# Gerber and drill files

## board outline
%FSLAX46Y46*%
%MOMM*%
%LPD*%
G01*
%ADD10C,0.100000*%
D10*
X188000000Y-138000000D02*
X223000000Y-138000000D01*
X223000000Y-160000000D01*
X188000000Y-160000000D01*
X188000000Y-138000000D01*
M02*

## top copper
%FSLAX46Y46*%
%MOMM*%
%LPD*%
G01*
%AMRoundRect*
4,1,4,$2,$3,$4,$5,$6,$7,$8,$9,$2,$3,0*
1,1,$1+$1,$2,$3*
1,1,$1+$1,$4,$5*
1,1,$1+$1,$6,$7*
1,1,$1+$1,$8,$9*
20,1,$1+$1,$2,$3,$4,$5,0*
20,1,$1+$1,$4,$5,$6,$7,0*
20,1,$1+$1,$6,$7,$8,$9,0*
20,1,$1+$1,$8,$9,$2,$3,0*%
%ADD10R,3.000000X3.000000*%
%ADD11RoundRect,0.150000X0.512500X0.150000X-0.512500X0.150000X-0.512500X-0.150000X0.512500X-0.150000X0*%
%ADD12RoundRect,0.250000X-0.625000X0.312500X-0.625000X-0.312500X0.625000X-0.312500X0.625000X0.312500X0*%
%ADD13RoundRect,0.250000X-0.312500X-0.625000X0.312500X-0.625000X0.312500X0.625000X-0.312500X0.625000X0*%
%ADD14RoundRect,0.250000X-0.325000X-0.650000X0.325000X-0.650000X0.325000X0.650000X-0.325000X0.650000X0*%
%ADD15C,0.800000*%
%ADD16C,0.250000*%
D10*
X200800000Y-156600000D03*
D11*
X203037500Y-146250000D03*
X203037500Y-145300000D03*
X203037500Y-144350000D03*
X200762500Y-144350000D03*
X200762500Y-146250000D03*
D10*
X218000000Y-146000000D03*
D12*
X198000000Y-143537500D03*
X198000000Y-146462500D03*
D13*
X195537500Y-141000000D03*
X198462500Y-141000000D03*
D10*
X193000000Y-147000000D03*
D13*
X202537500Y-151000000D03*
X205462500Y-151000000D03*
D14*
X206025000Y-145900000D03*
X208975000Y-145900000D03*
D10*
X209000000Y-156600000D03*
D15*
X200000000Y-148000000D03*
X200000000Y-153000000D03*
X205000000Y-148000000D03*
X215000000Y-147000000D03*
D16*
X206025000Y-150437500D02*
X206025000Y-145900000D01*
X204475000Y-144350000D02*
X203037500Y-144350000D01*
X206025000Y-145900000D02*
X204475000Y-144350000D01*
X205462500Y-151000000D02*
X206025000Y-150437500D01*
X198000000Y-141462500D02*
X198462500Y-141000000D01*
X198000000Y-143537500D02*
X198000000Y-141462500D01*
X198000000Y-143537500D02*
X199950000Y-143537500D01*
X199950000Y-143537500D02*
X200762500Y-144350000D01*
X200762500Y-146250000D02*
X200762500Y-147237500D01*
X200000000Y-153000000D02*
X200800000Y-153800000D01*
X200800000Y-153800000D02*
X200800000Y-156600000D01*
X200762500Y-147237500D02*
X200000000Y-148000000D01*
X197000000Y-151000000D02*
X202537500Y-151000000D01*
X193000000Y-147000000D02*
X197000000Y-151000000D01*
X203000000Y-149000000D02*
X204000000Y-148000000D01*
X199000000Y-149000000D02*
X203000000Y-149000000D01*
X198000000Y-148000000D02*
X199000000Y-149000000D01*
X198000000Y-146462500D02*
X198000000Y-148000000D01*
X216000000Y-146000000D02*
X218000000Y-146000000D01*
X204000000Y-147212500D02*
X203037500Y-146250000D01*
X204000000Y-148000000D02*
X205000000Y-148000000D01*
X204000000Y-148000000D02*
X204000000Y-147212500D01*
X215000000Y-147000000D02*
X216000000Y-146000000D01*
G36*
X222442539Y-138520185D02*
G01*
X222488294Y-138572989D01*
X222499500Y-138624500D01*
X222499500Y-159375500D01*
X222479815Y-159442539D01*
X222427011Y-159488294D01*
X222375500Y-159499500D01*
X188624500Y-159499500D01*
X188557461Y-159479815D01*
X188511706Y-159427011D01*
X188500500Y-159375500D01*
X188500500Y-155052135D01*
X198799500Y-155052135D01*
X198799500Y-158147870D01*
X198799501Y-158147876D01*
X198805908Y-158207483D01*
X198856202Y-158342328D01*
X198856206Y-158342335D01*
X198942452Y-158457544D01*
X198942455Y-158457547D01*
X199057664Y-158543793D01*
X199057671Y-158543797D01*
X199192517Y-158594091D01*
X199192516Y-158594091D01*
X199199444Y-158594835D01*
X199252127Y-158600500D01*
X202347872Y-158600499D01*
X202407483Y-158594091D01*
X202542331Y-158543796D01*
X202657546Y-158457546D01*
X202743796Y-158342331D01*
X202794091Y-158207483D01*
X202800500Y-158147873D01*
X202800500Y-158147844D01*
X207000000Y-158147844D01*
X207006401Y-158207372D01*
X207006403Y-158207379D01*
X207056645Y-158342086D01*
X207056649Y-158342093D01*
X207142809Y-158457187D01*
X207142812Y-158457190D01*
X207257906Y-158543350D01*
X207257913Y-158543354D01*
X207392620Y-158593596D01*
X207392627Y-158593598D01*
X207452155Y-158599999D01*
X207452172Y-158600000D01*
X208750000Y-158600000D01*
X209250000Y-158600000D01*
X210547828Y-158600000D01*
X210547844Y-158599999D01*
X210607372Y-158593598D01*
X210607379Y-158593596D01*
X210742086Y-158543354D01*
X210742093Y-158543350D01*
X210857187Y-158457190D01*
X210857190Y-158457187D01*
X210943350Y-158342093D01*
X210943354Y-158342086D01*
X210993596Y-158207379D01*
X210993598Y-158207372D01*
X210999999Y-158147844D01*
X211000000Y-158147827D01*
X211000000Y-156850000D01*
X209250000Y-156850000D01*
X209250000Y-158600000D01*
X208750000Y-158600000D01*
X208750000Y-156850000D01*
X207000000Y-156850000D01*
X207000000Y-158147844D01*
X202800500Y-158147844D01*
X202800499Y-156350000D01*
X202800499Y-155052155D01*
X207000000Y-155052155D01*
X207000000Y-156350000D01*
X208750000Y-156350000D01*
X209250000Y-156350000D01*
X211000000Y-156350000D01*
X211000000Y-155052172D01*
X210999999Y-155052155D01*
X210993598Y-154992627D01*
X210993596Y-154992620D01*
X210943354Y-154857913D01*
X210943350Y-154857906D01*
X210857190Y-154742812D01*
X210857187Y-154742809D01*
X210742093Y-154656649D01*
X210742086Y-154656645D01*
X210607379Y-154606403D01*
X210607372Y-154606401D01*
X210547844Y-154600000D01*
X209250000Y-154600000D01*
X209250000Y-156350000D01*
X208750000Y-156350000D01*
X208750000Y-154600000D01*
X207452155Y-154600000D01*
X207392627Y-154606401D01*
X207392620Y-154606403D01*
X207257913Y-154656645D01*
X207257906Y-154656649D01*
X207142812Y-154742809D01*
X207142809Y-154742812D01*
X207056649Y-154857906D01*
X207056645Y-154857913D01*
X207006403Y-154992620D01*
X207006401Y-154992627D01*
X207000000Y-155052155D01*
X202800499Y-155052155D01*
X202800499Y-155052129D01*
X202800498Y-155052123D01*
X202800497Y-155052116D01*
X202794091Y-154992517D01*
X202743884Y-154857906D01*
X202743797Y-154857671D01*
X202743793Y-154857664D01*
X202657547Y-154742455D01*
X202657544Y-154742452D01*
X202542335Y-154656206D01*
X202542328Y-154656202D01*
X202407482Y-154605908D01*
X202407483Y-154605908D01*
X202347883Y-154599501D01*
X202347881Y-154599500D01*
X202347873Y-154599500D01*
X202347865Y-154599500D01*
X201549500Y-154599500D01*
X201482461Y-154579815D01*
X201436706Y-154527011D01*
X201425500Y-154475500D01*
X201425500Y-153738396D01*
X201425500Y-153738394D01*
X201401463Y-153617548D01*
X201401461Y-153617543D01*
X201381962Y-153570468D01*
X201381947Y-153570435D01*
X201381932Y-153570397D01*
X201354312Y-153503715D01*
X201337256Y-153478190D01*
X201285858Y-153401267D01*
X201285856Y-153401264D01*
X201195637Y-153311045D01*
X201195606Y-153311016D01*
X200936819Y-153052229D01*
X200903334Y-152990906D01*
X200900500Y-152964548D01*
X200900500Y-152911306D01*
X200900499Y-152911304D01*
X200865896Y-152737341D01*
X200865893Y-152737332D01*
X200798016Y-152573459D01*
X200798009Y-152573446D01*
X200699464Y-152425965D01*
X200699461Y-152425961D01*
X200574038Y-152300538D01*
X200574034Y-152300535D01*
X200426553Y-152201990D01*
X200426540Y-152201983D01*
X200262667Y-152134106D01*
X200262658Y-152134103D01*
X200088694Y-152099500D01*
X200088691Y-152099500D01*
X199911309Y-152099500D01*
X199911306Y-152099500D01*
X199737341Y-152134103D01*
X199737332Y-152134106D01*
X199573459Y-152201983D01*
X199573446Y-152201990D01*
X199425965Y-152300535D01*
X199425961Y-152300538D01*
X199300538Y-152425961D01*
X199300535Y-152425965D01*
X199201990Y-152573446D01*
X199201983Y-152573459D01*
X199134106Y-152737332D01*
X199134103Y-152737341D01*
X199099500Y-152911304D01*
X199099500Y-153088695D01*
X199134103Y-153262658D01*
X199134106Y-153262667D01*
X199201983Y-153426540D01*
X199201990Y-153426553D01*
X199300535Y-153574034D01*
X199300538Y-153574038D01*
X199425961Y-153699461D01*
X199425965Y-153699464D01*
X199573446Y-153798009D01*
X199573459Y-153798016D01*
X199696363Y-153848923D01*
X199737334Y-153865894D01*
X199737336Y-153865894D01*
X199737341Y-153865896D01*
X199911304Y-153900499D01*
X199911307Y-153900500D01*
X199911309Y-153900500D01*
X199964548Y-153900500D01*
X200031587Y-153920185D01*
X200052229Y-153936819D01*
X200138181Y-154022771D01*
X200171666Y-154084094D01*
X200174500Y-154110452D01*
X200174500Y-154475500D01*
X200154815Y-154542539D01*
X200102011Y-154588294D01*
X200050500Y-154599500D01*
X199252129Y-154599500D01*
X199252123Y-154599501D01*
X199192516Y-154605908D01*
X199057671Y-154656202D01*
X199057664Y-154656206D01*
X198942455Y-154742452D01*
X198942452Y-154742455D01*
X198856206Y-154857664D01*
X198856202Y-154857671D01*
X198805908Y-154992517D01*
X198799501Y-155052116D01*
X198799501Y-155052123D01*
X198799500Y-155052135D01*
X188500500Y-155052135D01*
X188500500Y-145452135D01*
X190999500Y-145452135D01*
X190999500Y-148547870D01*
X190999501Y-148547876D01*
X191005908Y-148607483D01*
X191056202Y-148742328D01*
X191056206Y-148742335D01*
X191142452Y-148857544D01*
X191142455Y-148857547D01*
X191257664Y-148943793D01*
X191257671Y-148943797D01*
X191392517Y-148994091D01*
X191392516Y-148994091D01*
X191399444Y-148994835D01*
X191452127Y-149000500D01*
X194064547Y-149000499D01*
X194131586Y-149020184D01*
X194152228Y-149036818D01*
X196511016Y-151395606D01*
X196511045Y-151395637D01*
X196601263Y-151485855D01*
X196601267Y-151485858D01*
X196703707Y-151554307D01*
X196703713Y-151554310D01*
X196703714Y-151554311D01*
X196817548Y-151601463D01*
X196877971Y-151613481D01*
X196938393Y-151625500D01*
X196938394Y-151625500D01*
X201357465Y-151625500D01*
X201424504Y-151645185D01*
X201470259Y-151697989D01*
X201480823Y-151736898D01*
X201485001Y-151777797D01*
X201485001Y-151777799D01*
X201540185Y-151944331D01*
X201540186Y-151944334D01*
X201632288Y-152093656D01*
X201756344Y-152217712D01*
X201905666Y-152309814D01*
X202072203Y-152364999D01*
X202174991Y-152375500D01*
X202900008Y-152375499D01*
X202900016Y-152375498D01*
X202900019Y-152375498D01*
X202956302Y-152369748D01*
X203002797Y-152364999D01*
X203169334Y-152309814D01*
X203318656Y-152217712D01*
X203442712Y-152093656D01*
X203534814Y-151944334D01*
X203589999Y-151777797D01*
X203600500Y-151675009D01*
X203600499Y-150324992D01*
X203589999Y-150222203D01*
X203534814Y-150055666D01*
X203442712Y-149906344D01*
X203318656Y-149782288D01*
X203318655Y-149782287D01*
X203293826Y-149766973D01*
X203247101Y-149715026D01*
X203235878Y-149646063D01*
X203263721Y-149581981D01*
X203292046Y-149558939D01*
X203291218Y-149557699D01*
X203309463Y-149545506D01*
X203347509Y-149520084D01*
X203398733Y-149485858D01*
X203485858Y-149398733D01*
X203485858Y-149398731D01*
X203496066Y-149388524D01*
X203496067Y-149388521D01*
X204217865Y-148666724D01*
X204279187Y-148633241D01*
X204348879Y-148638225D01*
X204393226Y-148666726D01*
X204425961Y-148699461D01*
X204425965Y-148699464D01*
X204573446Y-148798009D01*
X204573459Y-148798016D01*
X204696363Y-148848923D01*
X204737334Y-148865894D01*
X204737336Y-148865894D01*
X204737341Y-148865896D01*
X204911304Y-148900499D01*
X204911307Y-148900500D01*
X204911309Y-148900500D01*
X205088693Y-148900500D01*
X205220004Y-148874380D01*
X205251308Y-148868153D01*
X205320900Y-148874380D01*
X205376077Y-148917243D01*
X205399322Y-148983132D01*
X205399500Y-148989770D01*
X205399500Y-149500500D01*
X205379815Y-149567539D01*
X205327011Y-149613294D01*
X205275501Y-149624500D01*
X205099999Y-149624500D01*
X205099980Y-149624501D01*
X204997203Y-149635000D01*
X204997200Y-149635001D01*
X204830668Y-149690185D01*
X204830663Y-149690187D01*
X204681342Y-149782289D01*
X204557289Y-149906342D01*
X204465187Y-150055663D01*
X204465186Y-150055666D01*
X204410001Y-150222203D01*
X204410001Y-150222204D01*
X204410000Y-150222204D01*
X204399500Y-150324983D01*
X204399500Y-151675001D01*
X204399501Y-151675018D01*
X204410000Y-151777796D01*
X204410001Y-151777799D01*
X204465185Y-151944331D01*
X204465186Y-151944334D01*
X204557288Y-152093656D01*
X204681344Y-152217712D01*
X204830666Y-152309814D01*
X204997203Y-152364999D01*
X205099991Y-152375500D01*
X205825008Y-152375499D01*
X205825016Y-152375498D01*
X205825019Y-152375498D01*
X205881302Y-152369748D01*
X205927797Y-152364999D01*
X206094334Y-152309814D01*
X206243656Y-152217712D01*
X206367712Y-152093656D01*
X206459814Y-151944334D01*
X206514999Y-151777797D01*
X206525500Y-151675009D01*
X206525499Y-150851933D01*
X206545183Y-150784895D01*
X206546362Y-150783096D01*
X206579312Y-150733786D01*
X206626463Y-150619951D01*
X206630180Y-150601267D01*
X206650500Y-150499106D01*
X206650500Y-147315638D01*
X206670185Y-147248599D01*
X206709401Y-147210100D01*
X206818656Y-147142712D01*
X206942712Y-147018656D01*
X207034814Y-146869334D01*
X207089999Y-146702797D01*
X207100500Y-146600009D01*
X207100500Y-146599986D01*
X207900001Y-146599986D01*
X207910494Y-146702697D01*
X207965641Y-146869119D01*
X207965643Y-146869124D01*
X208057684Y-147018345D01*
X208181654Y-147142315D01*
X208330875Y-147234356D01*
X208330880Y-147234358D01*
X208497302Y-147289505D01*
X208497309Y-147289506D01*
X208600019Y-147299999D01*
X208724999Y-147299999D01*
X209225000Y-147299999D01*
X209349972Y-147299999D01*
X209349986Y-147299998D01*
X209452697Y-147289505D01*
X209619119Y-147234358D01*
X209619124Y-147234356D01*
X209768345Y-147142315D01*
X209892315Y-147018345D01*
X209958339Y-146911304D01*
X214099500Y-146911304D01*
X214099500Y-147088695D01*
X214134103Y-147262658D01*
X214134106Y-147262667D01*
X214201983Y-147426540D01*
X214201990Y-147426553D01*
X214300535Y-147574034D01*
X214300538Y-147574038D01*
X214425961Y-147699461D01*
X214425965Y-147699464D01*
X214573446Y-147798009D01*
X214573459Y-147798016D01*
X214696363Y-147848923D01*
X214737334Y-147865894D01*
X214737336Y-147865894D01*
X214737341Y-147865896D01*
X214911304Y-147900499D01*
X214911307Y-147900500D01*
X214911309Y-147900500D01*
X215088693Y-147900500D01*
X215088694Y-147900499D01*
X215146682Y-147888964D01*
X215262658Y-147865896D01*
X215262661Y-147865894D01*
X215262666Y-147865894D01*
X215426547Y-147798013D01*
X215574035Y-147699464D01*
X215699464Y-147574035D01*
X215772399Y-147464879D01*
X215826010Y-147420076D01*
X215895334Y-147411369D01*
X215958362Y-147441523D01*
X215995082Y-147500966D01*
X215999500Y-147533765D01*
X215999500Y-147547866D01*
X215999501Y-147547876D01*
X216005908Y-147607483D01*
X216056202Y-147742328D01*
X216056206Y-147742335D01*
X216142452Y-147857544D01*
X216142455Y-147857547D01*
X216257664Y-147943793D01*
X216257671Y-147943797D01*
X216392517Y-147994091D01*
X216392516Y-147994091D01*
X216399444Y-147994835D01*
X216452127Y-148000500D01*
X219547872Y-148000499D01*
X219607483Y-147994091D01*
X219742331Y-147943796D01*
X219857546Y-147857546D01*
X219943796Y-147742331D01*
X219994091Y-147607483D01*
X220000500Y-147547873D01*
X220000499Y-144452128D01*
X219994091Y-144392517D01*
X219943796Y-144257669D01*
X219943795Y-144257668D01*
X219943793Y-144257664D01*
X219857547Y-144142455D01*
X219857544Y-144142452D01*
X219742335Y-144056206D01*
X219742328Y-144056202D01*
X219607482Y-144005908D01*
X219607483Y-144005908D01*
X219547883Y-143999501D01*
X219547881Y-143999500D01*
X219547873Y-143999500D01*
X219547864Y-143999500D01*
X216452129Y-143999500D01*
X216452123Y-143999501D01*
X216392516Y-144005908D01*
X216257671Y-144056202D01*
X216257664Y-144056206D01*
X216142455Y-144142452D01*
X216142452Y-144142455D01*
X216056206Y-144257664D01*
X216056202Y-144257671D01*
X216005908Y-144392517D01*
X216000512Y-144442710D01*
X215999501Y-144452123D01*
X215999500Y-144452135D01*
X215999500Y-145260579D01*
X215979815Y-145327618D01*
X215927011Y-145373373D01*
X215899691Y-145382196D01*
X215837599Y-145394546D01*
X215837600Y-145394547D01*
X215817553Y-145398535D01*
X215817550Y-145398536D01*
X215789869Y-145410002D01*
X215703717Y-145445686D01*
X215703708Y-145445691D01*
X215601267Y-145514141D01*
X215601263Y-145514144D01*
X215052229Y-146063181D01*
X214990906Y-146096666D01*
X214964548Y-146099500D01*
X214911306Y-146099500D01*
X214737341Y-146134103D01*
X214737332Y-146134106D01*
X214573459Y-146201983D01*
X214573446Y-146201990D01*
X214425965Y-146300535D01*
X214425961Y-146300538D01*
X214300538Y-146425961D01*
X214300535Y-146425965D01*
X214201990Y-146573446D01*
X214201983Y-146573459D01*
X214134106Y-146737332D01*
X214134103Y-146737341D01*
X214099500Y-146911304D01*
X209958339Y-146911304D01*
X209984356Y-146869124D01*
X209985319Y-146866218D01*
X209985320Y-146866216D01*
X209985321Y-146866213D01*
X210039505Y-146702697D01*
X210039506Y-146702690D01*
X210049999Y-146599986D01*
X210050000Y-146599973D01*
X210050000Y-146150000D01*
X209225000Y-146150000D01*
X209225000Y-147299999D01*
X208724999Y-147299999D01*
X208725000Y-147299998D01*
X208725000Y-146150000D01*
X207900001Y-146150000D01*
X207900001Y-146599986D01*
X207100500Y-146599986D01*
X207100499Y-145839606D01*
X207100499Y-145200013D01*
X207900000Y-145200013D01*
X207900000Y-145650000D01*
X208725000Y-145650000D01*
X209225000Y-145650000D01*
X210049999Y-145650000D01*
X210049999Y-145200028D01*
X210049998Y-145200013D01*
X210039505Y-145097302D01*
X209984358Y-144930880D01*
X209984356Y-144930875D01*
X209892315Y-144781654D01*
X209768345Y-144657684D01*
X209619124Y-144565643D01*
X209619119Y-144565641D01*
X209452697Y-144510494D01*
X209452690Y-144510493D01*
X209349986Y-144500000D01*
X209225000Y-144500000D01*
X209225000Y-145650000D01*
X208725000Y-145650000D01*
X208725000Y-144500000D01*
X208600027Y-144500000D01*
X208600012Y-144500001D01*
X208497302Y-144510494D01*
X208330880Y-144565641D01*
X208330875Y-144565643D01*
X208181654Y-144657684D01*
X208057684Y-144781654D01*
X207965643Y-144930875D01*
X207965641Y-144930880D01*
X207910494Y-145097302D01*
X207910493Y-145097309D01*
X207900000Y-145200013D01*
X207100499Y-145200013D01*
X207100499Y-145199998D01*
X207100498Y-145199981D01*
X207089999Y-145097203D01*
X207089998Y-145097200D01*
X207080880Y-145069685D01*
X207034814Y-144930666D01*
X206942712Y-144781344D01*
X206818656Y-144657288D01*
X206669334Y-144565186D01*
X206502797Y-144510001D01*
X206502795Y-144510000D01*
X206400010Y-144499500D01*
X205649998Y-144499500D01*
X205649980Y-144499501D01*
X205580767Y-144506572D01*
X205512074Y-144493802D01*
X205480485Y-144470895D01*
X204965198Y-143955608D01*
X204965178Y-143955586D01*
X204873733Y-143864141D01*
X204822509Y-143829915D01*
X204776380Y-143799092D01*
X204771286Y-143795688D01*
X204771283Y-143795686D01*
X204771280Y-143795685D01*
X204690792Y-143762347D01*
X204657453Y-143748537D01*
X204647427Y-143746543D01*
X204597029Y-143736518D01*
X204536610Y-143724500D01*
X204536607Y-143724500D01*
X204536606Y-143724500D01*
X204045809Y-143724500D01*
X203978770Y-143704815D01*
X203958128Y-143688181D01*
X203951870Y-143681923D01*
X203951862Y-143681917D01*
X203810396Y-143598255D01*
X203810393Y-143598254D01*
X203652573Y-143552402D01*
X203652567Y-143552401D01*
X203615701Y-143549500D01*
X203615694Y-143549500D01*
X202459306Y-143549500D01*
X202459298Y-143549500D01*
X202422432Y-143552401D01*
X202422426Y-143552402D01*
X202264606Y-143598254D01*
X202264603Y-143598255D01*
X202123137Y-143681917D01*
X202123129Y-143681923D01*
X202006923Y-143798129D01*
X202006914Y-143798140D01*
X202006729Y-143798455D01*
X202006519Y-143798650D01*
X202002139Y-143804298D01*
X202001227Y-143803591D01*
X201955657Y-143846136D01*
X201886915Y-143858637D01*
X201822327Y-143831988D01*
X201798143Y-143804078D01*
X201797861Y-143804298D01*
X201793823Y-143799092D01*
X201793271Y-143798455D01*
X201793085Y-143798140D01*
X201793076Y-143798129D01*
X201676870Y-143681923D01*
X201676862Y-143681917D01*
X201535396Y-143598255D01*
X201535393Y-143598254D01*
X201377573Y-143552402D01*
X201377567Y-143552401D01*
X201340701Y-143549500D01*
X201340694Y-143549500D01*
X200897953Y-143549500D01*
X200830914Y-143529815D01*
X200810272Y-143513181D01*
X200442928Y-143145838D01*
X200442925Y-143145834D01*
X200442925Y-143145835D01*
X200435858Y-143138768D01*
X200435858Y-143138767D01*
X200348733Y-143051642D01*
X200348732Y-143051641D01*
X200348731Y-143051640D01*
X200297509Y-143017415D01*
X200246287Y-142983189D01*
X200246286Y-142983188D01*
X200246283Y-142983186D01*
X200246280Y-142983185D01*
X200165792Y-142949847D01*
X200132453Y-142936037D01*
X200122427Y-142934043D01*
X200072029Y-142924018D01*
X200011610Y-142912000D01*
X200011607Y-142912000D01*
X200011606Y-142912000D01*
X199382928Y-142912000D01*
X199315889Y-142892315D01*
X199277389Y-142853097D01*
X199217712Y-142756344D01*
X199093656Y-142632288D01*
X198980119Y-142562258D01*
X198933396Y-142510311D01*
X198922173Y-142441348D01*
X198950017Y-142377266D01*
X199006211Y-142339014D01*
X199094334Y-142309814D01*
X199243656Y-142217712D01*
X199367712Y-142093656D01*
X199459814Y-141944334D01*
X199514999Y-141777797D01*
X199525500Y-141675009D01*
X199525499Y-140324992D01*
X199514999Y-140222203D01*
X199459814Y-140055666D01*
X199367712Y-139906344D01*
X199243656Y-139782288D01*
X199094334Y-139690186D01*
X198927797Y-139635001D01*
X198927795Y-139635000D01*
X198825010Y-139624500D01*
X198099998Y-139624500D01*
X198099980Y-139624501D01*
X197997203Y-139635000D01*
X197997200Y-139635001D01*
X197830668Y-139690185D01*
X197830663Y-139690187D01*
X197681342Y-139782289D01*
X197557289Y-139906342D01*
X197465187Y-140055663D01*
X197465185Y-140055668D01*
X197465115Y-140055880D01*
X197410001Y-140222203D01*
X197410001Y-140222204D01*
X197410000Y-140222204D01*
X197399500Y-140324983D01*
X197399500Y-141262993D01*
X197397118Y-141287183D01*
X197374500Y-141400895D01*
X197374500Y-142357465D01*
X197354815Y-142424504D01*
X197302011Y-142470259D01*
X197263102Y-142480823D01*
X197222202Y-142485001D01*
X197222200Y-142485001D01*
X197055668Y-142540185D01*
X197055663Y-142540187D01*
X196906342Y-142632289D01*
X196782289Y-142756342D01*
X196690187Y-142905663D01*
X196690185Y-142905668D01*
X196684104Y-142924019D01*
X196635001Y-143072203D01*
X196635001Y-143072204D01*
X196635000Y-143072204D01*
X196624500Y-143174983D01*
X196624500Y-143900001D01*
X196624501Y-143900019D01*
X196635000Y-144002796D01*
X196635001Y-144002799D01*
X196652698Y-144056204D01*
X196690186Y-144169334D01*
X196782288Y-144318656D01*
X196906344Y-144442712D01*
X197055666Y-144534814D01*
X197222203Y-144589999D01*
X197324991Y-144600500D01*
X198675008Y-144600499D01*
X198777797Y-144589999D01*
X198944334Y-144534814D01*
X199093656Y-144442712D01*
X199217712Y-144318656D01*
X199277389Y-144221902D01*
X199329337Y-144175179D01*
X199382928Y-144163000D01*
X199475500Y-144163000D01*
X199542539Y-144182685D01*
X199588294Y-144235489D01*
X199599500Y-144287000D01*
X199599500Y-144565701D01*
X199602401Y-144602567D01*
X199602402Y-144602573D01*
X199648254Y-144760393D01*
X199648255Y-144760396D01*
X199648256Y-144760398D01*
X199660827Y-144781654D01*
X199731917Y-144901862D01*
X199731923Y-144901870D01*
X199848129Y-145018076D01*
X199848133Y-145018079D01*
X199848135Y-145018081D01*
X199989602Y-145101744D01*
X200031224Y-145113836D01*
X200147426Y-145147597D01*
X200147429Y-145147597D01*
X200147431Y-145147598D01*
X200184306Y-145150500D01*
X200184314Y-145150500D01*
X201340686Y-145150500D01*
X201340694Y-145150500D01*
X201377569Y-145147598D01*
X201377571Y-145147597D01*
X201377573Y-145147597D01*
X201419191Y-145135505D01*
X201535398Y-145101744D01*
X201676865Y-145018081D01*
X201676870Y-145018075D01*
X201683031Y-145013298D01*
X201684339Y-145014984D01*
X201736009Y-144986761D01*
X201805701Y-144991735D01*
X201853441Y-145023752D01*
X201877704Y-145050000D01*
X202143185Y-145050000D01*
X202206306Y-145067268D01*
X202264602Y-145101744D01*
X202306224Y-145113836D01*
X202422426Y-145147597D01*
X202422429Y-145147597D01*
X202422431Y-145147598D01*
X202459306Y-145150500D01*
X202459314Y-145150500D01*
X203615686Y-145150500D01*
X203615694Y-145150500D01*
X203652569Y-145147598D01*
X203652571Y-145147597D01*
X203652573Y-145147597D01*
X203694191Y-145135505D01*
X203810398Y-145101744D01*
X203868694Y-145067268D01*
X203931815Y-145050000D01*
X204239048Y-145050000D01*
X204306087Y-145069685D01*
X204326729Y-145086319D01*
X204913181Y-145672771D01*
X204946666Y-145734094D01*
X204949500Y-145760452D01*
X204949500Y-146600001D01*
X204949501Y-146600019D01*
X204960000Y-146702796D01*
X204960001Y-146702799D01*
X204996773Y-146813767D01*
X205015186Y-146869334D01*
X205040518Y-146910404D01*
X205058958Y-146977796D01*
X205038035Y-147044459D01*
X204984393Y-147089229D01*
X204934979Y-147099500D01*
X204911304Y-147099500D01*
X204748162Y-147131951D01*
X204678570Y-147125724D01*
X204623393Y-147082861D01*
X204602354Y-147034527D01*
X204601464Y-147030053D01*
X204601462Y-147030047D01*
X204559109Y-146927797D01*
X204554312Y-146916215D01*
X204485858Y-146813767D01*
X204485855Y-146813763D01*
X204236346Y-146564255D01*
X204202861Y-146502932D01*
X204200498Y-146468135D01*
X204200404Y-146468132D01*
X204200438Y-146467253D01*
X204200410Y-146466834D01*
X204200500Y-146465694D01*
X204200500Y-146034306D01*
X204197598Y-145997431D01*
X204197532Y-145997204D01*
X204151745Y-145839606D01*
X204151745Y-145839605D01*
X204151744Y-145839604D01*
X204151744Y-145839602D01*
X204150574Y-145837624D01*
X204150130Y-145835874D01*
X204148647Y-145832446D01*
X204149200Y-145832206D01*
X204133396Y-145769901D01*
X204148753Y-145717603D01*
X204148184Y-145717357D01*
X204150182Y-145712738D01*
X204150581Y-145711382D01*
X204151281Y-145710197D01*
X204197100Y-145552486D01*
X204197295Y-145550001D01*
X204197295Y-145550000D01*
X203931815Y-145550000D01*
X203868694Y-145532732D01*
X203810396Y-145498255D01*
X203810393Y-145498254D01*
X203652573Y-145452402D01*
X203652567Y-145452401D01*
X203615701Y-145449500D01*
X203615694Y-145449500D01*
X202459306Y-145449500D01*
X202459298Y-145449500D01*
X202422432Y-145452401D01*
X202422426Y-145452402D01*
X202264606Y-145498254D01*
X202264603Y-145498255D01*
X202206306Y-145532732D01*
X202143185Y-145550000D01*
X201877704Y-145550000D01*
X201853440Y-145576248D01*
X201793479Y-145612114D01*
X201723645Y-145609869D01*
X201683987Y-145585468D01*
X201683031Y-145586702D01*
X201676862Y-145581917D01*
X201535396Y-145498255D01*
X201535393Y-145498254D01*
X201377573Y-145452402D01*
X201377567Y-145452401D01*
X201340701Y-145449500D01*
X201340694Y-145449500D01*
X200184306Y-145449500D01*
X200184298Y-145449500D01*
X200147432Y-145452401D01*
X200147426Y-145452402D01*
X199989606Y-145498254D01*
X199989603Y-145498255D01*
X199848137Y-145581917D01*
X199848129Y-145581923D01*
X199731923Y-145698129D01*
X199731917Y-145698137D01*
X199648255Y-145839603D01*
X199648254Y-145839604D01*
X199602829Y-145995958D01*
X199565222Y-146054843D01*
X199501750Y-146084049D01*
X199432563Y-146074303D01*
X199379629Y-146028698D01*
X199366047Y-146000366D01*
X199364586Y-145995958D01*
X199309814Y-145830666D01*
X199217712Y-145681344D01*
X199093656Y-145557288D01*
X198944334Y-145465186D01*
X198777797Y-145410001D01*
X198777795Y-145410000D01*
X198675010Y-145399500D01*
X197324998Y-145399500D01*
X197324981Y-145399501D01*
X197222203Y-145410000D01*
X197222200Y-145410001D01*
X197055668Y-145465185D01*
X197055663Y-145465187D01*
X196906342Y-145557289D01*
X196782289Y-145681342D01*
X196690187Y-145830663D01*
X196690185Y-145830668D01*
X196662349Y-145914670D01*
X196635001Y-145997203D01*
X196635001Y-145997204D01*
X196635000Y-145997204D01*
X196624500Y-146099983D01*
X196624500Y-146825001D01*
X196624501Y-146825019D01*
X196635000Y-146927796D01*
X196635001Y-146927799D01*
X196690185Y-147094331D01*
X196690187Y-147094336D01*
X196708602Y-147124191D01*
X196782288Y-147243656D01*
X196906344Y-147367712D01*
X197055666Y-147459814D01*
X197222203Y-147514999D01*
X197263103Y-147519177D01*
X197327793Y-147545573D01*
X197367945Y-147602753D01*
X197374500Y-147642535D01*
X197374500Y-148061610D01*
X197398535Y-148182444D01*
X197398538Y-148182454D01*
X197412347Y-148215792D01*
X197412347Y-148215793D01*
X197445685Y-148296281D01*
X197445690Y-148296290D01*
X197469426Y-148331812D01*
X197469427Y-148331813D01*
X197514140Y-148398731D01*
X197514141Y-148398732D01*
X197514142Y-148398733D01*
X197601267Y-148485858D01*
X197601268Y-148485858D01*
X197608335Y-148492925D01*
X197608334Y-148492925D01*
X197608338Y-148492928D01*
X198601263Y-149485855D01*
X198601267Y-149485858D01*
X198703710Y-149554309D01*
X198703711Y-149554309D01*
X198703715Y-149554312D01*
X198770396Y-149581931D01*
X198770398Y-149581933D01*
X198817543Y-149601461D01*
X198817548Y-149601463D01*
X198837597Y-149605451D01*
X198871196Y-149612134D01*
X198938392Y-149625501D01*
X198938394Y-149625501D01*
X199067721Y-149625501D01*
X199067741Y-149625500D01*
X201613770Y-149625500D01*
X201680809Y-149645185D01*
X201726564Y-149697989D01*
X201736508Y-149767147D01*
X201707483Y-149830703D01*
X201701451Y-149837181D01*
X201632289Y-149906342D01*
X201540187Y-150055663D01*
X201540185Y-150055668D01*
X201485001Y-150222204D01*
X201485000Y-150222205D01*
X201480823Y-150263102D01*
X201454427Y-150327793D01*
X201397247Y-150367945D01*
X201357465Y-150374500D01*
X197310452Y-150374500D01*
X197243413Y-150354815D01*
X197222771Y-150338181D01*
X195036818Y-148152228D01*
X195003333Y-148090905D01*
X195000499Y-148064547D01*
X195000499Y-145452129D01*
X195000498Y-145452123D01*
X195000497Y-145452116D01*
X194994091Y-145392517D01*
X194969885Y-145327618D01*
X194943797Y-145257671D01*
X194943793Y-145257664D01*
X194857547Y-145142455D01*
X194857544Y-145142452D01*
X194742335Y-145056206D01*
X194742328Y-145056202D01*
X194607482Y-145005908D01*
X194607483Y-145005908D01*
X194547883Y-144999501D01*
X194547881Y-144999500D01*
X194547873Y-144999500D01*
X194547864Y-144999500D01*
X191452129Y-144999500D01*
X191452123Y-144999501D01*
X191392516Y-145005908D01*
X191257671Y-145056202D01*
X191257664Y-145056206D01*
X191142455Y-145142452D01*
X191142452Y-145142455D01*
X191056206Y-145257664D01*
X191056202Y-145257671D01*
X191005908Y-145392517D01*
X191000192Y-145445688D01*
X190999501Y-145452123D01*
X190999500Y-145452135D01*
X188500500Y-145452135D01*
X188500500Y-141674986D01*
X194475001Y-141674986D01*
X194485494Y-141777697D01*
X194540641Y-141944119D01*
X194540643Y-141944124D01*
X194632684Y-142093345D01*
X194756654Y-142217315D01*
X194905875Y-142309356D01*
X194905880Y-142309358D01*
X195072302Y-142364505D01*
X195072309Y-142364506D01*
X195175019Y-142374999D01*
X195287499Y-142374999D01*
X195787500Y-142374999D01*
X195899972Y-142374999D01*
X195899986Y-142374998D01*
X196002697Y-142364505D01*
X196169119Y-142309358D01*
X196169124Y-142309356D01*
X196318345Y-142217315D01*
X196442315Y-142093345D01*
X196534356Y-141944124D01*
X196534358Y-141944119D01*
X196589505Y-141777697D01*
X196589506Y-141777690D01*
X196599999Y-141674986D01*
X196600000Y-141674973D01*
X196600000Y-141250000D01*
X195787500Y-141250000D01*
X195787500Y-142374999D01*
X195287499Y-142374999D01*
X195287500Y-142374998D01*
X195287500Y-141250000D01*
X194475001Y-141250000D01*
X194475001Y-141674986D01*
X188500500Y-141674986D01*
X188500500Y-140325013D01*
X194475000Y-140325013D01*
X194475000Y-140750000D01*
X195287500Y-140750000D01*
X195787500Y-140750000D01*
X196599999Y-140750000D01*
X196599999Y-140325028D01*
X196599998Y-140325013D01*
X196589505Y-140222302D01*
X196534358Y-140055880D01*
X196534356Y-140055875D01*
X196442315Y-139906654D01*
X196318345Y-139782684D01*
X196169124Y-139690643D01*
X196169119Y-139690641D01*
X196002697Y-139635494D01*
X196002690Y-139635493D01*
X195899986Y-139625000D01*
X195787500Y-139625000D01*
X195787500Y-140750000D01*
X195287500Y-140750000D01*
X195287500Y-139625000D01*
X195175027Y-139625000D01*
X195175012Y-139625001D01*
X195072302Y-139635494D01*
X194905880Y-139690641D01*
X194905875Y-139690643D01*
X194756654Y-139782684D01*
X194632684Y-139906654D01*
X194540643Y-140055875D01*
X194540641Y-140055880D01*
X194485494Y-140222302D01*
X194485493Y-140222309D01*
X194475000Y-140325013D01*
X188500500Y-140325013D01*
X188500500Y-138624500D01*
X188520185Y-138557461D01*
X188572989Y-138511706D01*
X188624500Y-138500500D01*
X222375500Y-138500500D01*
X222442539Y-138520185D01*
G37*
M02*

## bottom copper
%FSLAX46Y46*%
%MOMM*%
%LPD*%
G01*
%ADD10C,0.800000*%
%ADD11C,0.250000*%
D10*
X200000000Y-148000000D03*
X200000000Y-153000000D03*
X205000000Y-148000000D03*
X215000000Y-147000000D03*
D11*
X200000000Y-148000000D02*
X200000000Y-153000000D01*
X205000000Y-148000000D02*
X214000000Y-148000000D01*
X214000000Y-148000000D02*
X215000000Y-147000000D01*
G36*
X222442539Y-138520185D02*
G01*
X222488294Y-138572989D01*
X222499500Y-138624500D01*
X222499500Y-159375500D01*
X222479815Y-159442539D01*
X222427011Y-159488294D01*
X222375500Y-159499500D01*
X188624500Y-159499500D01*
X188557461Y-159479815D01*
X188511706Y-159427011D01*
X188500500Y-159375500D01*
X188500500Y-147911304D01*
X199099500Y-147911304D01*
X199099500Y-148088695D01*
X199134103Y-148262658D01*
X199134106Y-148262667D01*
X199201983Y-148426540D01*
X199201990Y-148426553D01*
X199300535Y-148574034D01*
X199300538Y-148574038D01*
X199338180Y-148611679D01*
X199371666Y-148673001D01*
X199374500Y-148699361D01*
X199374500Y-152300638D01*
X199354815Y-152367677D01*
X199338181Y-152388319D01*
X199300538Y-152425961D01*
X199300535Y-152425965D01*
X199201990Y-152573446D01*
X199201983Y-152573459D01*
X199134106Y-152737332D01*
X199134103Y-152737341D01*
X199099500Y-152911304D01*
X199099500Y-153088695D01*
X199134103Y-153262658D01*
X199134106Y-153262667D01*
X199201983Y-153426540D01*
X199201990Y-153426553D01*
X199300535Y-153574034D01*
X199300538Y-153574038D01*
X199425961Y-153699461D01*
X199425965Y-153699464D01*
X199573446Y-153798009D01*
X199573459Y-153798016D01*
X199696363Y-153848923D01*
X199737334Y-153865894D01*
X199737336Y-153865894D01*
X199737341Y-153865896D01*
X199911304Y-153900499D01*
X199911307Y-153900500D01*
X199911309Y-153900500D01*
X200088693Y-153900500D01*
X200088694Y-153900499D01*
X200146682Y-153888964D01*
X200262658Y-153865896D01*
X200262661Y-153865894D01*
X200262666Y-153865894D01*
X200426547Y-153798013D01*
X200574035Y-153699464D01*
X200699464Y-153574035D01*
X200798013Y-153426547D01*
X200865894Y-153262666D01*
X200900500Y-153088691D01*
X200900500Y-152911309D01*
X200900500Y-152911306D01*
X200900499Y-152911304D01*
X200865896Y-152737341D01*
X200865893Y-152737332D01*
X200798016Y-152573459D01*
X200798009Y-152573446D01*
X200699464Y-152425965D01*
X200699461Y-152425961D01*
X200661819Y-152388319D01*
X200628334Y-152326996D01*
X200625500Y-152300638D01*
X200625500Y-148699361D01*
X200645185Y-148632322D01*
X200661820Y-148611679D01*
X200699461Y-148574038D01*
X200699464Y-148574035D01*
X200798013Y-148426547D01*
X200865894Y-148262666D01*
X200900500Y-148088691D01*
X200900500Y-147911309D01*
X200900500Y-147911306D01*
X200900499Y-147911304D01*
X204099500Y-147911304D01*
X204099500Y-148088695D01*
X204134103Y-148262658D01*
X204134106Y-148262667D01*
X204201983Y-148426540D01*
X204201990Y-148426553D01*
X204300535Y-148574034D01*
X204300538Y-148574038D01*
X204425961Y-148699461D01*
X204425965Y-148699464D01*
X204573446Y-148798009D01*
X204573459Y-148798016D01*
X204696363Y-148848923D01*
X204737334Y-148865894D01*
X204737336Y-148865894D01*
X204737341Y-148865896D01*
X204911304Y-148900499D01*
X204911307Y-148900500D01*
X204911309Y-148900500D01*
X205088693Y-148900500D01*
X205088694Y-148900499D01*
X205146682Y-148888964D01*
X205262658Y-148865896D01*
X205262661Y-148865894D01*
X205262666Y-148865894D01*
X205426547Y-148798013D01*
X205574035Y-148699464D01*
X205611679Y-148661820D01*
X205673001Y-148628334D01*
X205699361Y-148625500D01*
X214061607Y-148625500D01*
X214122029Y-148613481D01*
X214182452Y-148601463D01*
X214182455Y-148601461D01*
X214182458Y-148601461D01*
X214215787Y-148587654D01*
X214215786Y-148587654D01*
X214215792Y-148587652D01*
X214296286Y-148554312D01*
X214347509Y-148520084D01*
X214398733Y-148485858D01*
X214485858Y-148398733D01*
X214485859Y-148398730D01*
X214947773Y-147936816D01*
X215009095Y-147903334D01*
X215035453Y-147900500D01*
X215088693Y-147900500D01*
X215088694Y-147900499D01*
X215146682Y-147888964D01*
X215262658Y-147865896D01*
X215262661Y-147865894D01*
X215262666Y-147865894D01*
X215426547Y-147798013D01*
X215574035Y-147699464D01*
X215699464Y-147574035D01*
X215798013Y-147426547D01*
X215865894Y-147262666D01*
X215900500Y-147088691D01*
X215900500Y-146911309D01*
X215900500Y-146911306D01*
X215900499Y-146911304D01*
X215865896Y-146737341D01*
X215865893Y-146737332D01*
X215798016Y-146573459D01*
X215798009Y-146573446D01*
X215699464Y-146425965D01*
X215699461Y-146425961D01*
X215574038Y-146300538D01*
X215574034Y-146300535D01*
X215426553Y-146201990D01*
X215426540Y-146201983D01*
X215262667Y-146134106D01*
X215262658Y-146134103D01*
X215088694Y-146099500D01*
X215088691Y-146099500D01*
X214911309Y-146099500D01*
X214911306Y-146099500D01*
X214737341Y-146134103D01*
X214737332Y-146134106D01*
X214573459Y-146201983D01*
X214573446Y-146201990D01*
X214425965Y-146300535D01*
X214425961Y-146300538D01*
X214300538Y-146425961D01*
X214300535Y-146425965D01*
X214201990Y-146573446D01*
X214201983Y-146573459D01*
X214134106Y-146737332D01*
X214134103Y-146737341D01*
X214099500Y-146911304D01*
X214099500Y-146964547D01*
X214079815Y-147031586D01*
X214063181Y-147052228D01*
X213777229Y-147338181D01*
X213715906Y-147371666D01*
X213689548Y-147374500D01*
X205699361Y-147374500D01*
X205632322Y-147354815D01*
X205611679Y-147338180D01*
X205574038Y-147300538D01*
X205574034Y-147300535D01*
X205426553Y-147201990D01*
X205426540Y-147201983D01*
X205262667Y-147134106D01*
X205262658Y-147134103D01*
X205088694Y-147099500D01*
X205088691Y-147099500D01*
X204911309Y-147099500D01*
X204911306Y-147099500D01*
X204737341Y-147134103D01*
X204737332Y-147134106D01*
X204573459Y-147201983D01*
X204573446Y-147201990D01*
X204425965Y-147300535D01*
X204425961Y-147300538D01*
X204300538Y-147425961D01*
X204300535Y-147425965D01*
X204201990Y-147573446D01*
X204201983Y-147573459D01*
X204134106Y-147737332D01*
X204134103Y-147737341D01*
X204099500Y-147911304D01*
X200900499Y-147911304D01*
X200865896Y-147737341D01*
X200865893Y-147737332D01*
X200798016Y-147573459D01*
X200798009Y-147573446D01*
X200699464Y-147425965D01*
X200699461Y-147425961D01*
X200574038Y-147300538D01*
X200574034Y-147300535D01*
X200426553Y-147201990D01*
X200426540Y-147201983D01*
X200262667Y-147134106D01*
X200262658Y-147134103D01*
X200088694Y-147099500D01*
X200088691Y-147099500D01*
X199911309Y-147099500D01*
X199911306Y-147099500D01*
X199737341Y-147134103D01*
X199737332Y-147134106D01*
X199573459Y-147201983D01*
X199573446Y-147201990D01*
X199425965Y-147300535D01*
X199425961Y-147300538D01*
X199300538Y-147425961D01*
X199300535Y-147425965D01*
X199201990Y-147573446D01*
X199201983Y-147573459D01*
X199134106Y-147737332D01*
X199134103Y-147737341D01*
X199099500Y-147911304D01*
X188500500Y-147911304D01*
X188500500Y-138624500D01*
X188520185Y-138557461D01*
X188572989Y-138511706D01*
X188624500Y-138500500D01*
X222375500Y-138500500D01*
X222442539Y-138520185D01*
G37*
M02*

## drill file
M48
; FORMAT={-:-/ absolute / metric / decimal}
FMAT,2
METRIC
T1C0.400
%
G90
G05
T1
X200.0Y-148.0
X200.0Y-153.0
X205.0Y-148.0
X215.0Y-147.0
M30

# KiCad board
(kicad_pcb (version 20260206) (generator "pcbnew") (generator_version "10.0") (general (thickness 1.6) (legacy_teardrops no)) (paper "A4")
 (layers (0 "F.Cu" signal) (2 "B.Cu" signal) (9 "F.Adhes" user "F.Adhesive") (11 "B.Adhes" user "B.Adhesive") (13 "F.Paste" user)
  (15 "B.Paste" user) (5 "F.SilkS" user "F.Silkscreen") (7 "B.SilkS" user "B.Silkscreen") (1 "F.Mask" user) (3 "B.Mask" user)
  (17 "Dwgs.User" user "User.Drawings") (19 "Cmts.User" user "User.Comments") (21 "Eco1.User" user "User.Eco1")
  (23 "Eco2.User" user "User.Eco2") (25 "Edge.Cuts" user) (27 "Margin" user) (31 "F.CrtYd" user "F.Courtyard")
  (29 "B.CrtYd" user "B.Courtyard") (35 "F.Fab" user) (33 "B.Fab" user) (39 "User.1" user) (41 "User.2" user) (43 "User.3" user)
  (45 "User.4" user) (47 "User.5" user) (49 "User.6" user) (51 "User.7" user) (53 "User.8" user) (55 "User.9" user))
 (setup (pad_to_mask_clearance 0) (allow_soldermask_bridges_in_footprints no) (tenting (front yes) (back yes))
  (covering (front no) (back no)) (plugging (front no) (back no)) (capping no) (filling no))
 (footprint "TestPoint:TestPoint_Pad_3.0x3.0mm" (layer "F.Cu") (at 200.8 156.6)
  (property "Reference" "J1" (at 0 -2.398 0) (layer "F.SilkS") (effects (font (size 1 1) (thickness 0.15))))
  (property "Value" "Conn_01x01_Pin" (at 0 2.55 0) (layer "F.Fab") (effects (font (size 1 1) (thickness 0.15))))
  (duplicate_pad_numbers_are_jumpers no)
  (pad "1" smd rect (at 0 0) (size 3 3) (layers "F.Cu" "F.Mask") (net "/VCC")))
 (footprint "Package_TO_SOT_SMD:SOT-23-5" (layer "F.Cu") (at 201.9 145.3 180)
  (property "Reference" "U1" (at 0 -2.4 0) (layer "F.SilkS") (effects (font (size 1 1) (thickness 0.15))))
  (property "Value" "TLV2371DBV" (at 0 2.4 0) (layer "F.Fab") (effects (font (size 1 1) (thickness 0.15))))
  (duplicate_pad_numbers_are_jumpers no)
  (pad "1" smd roundrect (at -1.1375 -0.95 180) (size 1.325 0.6) (layers "F.Cu" "F.Mask" "F.Paste") (roundrect_rratio 0.25) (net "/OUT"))
  (pad "2" smd roundrect (at -1.1375 0 180) (size 1.325 0.6) (layers "F.Cu" "F.Mask" "F.Paste") (roundrect_rratio 0.25) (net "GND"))
  (pad "3" smd roundrect (at -1.1375 0.95 180) (size 1.325 0.6) (layers "F.Cu" "F.Mask" "F.Paste") (roundrect_rratio 0.25)
   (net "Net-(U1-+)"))
  (pad "4" smd roundrect (at 1.1375 0.95 180) (size 1.325 0.6) (layers "F.Cu" "F.Mask" "F.Paste") (roundrect_rratio 0.25) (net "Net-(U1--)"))
  (pad "5" smd roundrect (at 1.1375 -0.95 180) (size 1.325 0.6) (layers "F.Cu" "F.Mask" "F.Paste") (roundrect_rratio 0.25) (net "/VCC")))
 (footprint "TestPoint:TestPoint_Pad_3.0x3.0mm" (layer "F.Cu") (at 218 146)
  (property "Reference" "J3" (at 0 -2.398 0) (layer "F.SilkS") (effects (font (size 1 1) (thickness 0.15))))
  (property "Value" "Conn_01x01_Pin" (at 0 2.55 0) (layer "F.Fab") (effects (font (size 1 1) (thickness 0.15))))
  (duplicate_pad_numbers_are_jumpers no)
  (pad "1" smd rect (at 0 0) (size 3 3) (layers "F.Cu" "F.Mask") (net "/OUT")))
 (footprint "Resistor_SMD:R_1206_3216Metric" (layer "F.Cu") (at 198 145 -90)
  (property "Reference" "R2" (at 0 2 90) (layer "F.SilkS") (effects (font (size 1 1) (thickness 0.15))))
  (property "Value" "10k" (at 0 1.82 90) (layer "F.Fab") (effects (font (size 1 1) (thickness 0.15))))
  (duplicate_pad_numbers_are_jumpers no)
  (pad "1" smd roundrect (at -1.4625 0 270) (size 1.125 1.75) (layers "F.Cu" "F.Mask" "F.Paste") (roundrect_rratio 0.222222)
   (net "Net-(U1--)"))
  (pad "2" smd roundrect (at 1.4625 0 270) (size 1.125 1.75) (layers "F.Cu" "F.Mask" "F.Paste") (roundrect_rratio 0.222222) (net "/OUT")))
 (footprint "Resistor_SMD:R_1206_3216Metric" (layer "F.Cu") (at 197 141)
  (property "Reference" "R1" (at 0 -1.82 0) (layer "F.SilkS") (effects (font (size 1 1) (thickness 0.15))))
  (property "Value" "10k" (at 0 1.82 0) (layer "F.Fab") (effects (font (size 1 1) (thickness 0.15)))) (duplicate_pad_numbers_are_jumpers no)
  (pad "1" smd roundrect (at -1.4625 0) (size 1.125 1.75) (layers "F.Cu" "F.Mask" "F.Paste") (roundrect_rratio 0.222222) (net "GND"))
  (pad "2" smd roundrect (at 1.4625 0) (size 1.125 1.75) (layers "F.Cu" "F.Mask" "F.Paste") (roundrect_rratio 0.222222) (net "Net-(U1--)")))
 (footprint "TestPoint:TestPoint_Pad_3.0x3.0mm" (layer "F.Cu") (at 193 147)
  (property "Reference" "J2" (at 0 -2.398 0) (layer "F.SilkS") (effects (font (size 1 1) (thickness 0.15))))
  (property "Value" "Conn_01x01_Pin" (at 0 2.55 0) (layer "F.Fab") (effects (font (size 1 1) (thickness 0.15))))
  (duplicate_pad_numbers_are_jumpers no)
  (pad "1" smd rect (at 0 0) (size 3 3) (layers "F.Cu" "F.Mask") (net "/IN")))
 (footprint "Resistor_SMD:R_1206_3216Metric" (layer "F.Cu") (at 204 151)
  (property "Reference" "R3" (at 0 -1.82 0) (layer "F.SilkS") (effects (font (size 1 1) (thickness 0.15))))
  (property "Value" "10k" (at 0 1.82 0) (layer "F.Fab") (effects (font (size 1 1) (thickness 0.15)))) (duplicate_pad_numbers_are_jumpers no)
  (pad "1" smd roundrect (at -1.4625 0) (size 1.125 1.75) (layers "F.Cu" "F.Mask" "F.Paste") (roundrect_rratio 0.222222) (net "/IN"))
  (pad "2" smd roundrect (at 1.4625 0) (size 1.125 1.75) (layers "F.Cu" "F.Mask" "F.Paste") (roundrect_rratio 0.222222) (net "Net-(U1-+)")))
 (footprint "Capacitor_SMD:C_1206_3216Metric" (layer "F.Cu") (at 207.5 145.9)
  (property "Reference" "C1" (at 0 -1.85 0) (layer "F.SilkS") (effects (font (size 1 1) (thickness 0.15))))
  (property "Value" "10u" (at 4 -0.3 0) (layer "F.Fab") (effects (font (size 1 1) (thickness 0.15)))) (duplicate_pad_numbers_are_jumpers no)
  (pad "1" smd roundrect (at -1.475 0) (size 1.15 1.8) (layers "F.Cu" "F.Mask" "F.Paste") (roundrect_rratio 0.217391) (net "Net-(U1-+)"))
  (pad "2" smd roundrect (at 1.475 0) (size 1.15 1.8) (layers "F.Cu" "F.Mask" "F.Paste") (roundrect_rratio 0.217391) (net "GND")))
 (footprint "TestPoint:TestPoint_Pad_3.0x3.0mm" (layer "F.Cu") (at 209 156.6)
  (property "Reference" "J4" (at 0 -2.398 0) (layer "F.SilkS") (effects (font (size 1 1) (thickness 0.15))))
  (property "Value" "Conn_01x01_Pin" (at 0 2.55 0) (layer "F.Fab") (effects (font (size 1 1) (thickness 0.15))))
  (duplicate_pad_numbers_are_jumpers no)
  (pad "1" smd rect (at 0 0) (size 3 3) (layers "F.Cu" "F.Mask") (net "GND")))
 (gr_rect (start 188 138) (end 223 160) (stroke (width 0.1) (type default)) (fill no) (layer "Edge.Cuts"))
 (segment (start 206.025 150.4375) (end 206.025 145.9) (width 0.25) (layer "F.Cu") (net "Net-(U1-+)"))
 (segment (start 204.475 144.35) (end 203.0375 144.35) (width 0.25) (layer "F.Cu") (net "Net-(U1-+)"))
 (segment (start 206.025 145.9) (end 204.475 144.35) (width 0.25) (layer "F.Cu") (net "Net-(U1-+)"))
 (segment (start 205.4625 151) (end 206.025 150.4375) (width 0.25) (layer "F.Cu") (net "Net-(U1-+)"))
 (segment (start 198 141.4625) (end 198.4625 141) (width 0.25) (layer "F.Cu") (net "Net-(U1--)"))
 (segment (start 198 143.5375) (end 198 141.4625) (width 0.25) (layer "F.Cu") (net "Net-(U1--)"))
 (segment (start 198 143.5375) (end 199.95 143.5375) (width 0.25) (layer "F.Cu") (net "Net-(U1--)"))
 (segment (start 199.95 143.5375) (end 200.7625 144.35) (width 0.25) (layer "F.Cu") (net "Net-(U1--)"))
 (segment (start 200.7625 146.25) (end 200.7625 147.2375) (width 0.25) (layer "F.Cu") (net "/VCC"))
 (segment (start 200 153) (end 200.8 153.8) (width 0.25) (layer "F.Cu") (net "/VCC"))
 (segment (start 200.8 153.8) (end 200.8 156.6) (width 0.25) (layer "F.Cu") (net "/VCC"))
 (segment (start 200.7625 147.2375) (end 200 148) (width 0.25) (layer "F.Cu") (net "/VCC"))
 (via (at 200 148) (size 0.8) (drill 0.4) (layers "F.Cu" "B.Cu") (capping no) (covering (front no) (back no))
  (plugging (front no) (back no)) (filling no) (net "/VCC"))
 (via (at 200 153) (size 0.8) (drill 0.4) (layers "F.Cu" "B.Cu") (capping no) (covering (front no) (back no))
  (plugging (front no) (back no)) (filling no) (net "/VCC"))
 (segment (start 200 148) (end 200 153) (width 0.25) (layer "B.Cu") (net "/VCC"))
 (segment (start 197 151) (end 202.5375 151) (width 0.25) (layer "F.Cu") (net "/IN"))
 (segment (start 193 147) (end 197 151) (width 0.25) (layer "F.Cu") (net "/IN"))
 (segment (start 203 149) (end 204 148) (width 0.25) (layer "F.Cu") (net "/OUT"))
 (segment (start 199 149) (end 203 149) (width 0.25) (layer "F.Cu") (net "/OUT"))
 (segment (start 198 148) (end 199 149) (width 0.25) (layer "F.Cu") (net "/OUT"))
 (segment (start 198 146.4625) (end 198 148) (width 0.25) (layer "F.Cu") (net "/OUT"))
 (segment (start 216 146) (end 218 146) (width 0.25) (layer "F.Cu") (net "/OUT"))
 (segment (start 204 147.2125) (end 203.0375 146.25) (width 0.25) (layer "F.Cu") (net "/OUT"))
 (segment (start 204 148) (end 205 148) (width 0.25) (layer "F.Cu") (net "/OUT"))
 (segment (start 204 148) (end 204 147.2125) (width 0.25) (layer "F.Cu") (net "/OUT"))
 (segment (start 215 147) (end 216 146) (width 0.25) (layer "F.Cu") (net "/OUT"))
 (via (at 205 148) (size 0.8) (drill 0.4) (layers "F.Cu" "B.Cu") (capping no) (covering (front no) (back no))
  (plugging (front no) (back no)) (filling no) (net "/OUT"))
 (via (at 215 147) (size 0.8) (drill 0.4) (layers "F.Cu" "B.Cu") (capping no) (covering (front no) (back no))
  (plugging (front no) (back no)) (filling no) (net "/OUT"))
 (segment (start 205 148) (end 214 148) (width 0.25) (layer "B.Cu") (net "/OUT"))
 (segment (start 214 148) (end 215 147) (width 0.25) (layer "B.Cu") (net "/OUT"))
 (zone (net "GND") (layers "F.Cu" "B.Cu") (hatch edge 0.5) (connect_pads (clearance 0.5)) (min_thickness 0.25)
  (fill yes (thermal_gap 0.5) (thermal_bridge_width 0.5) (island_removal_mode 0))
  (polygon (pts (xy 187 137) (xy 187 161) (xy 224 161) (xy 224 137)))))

